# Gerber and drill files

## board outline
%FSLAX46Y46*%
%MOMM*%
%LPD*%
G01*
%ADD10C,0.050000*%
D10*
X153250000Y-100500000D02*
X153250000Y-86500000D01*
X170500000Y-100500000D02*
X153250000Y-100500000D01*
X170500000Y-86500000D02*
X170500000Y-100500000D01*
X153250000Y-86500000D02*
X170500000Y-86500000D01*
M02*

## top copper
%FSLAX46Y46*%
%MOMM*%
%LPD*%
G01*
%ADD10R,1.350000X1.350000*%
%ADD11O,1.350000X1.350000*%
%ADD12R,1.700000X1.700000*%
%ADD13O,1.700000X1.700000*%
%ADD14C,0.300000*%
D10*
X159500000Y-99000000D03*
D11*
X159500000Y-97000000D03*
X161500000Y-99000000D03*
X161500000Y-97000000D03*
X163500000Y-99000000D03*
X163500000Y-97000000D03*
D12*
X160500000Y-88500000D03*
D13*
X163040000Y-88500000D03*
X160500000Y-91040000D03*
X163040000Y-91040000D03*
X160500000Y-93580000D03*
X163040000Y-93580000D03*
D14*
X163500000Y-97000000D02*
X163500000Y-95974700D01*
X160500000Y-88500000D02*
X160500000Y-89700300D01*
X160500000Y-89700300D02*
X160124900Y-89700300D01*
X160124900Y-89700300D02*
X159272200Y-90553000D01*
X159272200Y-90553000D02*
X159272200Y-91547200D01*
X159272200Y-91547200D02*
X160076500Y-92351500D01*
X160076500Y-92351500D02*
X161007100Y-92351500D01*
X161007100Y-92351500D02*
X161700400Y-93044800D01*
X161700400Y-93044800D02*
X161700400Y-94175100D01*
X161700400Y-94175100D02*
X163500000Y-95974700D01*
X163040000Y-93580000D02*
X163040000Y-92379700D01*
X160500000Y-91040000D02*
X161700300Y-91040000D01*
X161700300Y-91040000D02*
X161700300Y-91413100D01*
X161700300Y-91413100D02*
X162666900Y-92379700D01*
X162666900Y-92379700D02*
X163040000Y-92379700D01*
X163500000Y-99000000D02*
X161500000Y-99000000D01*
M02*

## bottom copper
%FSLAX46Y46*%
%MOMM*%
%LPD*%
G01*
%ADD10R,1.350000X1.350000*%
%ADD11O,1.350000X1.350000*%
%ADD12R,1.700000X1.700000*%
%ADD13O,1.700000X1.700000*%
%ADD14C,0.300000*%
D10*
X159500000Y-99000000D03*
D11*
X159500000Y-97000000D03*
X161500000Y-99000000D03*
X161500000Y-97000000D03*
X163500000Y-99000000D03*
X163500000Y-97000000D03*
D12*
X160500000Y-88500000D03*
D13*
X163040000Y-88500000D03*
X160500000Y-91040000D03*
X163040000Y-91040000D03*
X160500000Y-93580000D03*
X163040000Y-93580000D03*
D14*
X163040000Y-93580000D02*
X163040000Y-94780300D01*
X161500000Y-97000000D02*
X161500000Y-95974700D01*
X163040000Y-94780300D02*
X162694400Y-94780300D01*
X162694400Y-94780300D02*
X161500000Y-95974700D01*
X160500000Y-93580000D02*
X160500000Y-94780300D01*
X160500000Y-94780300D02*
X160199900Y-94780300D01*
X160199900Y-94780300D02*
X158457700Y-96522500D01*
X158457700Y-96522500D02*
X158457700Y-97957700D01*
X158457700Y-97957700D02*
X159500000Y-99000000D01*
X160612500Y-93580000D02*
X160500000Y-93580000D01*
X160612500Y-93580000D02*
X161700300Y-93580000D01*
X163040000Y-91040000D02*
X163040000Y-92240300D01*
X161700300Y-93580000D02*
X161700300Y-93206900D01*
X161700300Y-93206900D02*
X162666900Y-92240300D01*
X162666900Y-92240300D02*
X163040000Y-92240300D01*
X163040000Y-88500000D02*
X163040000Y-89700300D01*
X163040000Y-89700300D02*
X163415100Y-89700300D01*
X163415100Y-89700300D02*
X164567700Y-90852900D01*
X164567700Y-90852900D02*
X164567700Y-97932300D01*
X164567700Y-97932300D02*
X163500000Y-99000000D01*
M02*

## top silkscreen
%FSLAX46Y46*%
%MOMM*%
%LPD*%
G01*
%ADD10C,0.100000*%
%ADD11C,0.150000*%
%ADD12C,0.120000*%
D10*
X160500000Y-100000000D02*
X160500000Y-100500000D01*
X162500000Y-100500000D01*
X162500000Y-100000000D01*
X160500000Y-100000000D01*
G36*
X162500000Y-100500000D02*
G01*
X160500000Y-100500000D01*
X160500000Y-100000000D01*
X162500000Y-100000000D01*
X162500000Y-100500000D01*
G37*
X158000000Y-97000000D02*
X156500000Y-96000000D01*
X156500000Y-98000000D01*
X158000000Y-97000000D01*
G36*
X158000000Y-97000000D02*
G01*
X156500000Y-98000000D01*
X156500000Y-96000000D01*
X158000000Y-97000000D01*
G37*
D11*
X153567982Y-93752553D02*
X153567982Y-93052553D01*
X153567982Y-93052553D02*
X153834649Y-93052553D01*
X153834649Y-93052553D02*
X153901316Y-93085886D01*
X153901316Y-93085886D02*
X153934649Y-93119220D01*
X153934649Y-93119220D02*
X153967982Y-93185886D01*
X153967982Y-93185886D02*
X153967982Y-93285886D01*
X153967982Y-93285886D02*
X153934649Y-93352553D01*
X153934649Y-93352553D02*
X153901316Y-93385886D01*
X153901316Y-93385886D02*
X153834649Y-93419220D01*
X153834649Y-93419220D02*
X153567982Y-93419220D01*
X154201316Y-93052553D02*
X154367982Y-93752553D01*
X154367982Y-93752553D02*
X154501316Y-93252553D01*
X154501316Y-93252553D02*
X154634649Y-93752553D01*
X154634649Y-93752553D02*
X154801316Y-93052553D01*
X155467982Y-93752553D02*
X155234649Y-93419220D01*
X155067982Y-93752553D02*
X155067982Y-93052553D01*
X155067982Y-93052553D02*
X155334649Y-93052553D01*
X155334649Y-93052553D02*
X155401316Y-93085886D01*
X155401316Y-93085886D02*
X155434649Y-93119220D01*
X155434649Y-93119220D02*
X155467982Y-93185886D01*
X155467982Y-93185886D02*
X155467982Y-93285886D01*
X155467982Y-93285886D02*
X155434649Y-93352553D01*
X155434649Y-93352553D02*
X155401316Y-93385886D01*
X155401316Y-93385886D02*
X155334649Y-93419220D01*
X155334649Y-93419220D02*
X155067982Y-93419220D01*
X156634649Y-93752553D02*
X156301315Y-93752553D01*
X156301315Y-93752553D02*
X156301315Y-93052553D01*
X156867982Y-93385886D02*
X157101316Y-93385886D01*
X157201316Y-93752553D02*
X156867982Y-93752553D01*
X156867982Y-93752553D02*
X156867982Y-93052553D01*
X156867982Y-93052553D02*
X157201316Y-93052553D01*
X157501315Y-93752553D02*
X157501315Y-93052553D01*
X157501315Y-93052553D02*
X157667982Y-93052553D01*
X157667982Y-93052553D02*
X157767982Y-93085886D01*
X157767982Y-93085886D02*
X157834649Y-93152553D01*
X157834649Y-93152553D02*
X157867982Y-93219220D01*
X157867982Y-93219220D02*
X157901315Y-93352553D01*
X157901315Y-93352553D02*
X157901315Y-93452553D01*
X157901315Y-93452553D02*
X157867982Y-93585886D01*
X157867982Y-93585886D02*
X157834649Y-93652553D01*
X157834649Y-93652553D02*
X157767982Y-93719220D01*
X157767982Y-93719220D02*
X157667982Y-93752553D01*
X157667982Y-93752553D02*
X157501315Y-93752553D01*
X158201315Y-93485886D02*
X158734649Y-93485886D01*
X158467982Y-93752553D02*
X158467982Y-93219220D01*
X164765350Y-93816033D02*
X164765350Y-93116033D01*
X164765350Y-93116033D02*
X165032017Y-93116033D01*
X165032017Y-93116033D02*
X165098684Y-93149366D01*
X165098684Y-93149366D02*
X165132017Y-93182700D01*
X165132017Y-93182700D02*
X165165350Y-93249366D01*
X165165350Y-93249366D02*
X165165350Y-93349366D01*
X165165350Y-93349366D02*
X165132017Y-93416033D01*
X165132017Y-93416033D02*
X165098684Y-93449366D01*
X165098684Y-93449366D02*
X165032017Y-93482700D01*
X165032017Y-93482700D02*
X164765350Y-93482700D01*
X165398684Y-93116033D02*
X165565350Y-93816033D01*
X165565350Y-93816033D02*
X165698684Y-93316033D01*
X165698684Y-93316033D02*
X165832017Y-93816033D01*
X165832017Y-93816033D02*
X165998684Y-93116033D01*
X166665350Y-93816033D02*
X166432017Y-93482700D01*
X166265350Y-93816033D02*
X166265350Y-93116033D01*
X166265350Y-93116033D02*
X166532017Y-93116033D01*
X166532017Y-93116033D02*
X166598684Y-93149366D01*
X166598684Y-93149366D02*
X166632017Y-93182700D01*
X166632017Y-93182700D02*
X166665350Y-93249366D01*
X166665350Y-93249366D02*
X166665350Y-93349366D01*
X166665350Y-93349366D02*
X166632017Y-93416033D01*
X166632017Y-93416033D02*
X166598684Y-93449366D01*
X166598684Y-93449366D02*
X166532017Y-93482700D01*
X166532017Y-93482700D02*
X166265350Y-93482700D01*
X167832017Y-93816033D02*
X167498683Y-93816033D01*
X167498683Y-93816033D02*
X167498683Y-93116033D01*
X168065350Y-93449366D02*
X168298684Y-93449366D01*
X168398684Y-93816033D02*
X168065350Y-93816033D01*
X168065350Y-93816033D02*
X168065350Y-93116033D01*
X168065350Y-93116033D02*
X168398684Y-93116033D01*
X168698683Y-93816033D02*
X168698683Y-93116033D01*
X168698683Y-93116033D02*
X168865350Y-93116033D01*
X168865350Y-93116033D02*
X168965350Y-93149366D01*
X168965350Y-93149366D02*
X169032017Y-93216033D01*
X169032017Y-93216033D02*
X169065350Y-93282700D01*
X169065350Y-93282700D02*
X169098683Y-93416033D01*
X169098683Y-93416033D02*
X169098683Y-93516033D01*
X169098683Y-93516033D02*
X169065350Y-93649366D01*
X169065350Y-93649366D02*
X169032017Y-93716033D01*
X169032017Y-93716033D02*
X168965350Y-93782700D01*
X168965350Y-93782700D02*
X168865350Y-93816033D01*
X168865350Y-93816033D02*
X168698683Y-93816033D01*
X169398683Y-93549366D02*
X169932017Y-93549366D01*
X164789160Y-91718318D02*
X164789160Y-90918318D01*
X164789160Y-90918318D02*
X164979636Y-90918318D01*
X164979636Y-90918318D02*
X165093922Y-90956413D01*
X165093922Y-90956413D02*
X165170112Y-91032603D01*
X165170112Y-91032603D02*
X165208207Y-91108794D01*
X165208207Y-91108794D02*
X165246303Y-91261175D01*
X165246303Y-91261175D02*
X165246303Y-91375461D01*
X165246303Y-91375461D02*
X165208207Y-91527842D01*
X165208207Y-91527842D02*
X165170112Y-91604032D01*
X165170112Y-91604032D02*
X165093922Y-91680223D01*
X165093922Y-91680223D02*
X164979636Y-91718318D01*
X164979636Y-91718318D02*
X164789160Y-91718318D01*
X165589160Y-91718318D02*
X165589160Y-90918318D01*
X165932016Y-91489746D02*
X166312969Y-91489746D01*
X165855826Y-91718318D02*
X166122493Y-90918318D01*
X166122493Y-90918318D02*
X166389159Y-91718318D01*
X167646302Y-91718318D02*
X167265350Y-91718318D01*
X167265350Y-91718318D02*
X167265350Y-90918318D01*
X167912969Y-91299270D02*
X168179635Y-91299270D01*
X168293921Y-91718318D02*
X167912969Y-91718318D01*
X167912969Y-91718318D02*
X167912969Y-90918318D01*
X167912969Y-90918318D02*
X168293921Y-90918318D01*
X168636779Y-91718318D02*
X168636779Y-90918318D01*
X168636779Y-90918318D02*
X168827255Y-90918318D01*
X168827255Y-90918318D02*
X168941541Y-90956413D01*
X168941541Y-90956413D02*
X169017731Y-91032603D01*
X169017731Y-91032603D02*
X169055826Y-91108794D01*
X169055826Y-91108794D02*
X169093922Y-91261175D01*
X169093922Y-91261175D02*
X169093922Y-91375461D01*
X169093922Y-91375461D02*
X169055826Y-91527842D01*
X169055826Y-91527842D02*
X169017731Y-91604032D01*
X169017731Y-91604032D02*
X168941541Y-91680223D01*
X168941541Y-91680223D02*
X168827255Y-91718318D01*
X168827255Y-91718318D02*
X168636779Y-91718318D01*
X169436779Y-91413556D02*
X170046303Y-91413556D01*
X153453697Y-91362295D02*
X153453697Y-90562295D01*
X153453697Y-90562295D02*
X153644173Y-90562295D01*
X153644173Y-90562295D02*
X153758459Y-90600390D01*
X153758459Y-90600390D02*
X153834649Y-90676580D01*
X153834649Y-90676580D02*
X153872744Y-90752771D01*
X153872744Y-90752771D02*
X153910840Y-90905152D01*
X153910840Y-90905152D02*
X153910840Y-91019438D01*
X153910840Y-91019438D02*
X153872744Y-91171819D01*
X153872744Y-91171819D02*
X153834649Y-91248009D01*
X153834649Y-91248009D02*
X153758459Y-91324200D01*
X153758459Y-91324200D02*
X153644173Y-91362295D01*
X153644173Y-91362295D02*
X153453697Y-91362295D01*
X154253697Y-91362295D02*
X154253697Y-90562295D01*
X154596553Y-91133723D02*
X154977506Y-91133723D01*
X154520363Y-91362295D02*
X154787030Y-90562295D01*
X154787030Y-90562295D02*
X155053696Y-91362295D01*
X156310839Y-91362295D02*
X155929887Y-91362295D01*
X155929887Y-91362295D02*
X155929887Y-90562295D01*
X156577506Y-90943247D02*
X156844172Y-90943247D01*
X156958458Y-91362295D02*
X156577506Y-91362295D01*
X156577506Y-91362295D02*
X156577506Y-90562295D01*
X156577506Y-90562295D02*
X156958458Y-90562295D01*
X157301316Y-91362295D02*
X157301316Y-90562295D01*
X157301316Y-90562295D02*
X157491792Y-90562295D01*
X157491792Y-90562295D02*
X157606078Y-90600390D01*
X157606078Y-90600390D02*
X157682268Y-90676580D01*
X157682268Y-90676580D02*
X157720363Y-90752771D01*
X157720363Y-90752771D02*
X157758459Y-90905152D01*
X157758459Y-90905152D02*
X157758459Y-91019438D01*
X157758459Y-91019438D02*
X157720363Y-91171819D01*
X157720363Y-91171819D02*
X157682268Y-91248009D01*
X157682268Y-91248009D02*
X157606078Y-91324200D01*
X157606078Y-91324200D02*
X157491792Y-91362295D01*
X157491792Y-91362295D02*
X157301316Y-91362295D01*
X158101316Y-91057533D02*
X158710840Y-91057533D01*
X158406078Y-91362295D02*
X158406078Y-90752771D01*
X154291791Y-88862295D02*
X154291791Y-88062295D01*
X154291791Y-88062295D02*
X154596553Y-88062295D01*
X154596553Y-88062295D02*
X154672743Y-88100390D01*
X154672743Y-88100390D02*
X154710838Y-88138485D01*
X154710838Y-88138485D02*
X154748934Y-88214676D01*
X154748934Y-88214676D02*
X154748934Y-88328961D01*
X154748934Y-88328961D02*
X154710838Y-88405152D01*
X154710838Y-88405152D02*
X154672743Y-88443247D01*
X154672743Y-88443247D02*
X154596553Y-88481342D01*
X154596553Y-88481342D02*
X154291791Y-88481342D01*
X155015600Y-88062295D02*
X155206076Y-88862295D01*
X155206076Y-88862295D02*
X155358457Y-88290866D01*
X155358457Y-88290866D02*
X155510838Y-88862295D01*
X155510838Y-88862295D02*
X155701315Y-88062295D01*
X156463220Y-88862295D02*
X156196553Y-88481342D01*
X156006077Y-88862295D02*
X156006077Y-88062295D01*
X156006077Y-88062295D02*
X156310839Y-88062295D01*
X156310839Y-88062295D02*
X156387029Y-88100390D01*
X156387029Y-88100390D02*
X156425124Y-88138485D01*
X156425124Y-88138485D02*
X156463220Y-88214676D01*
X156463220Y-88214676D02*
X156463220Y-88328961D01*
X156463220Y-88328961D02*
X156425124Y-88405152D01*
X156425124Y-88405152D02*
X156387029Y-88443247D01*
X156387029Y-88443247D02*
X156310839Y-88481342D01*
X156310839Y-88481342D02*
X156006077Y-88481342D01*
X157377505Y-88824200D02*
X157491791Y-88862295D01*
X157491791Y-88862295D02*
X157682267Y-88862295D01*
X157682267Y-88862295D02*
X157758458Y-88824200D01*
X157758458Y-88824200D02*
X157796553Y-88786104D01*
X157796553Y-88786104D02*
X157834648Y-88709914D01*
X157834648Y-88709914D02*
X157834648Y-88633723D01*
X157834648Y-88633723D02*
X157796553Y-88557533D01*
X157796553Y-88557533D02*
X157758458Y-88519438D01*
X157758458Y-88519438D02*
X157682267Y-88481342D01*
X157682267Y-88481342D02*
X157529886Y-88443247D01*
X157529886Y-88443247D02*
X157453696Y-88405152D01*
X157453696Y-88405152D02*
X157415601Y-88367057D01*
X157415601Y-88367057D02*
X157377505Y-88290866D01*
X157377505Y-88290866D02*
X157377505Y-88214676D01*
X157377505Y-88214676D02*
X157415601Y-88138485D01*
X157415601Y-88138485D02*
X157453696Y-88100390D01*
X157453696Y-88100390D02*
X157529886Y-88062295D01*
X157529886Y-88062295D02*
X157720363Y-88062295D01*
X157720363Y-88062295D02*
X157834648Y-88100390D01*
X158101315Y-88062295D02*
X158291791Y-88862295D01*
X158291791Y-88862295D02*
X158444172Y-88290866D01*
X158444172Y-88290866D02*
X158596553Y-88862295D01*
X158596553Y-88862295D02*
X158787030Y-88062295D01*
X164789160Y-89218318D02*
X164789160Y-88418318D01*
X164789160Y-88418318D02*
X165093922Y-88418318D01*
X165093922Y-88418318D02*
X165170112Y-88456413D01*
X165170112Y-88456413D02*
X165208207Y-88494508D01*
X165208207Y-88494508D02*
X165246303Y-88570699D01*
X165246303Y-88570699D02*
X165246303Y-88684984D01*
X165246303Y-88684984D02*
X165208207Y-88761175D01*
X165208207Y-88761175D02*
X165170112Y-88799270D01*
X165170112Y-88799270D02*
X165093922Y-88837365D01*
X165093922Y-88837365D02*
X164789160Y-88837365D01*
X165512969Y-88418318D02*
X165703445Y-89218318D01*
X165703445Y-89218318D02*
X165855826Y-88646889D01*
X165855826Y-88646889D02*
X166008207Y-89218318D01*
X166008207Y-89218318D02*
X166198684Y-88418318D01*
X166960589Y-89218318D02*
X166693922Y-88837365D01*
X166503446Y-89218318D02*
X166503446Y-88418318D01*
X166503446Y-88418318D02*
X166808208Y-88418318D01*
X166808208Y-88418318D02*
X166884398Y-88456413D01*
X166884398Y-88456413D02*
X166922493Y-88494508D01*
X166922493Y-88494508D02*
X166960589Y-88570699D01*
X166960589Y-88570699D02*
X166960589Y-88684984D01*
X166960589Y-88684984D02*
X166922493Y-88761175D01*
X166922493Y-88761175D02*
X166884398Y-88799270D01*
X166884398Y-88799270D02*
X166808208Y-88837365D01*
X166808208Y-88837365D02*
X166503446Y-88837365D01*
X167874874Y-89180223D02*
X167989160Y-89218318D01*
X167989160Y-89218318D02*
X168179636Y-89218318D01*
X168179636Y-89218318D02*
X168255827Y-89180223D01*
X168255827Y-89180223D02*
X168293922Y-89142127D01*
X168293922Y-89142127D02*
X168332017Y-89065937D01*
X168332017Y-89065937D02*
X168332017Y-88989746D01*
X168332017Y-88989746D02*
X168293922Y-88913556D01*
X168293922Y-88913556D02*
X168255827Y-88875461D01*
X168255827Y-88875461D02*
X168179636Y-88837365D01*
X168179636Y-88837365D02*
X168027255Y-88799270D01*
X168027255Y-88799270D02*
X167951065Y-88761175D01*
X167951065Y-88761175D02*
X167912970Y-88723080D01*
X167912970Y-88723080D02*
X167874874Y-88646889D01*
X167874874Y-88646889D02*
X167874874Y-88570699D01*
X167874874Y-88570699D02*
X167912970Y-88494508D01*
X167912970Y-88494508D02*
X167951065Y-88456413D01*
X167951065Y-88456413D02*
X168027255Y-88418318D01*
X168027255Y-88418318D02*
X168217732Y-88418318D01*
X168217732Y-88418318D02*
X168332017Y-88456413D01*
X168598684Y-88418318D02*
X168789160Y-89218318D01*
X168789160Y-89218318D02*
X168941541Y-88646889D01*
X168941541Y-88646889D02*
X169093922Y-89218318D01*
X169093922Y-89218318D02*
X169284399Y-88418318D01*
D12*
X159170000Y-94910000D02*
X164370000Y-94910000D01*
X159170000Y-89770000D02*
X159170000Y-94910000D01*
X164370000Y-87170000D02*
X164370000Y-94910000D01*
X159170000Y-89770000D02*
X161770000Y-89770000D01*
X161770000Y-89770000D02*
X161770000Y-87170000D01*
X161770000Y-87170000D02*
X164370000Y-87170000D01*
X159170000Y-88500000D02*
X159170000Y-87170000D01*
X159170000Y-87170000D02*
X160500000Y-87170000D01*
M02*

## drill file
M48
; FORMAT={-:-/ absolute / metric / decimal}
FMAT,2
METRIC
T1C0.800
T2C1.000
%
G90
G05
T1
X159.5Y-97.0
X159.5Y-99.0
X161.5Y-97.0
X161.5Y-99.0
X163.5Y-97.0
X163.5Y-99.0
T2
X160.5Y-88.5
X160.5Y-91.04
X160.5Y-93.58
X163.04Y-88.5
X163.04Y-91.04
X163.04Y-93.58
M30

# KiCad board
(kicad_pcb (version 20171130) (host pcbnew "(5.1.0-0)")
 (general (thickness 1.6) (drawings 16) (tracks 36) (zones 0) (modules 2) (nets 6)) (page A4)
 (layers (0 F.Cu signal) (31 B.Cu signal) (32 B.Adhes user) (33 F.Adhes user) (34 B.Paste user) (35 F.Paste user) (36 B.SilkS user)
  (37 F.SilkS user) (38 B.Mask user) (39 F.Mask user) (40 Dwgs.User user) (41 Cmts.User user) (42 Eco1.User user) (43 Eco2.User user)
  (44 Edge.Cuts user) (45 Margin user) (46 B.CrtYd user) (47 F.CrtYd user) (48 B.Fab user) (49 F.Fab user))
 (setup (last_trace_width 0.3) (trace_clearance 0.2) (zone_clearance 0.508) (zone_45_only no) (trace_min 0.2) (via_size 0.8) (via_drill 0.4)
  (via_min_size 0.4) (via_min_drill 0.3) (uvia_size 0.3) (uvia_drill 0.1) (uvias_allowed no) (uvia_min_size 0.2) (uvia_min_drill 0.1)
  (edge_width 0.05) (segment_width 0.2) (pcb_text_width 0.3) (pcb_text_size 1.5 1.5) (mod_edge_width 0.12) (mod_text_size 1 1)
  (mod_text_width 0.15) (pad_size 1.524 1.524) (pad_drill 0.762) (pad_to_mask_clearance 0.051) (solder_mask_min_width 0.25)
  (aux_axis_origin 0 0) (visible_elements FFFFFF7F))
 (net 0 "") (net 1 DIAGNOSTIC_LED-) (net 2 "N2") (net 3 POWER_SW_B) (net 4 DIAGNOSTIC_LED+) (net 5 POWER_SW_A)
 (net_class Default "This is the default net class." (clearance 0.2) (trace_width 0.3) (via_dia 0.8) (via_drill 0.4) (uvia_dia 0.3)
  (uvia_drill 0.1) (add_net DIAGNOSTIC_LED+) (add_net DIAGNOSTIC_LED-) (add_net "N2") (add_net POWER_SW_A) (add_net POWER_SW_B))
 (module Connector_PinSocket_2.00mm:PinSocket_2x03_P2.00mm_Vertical (layer B.Cu) (at 159.5 99 270)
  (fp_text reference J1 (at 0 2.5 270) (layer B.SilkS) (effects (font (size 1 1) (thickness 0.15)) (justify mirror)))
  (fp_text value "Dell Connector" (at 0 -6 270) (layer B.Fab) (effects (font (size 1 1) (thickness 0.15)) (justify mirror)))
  (pad 1 thru_hole rect (at 0 0 270) (size 1.35 1.35) (drill 0.8) (layers *.Cu *.Mask) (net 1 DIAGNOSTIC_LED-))
  (pad 2 thru_hole oval (at -2 0 270) (size 1.35 1.35) (drill 0.8) (layers *.Cu *.Mask) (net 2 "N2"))
  (pad 3 thru_hole oval (at 0 -2 270) (size 1.35 1.35) (drill 0.8) (layers *.Cu *.Mask) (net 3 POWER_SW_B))
  (pad 4 thru_hole oval (at -2 -2 270) (size 1.35 1.35) (drill 0.8) (layers *.Cu *.Mask) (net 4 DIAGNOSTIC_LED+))
  (pad 5 thru_hole oval (at 0 -4 270) (size 1.35 1.35) (drill 0.8) (layers *.Cu *.Mask) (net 3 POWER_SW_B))
  (pad 6 thru_hole oval (at -2 -4 270) (size 1.35 1.35) (drill 0.8) (layers *.Cu *.Mask) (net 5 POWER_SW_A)))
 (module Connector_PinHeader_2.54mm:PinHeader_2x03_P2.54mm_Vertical (layer F.Cu) (at 160.5 88.5)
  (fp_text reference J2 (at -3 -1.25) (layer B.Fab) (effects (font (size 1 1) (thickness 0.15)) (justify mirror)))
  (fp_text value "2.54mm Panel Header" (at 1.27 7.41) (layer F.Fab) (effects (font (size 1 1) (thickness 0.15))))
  (fp_line (start -1.33 6.41) (end 3.87 6.41) (layer F.SilkS) (width 0.12))
  (fp_line (start -1.33 1.27) (end -1.33 6.41) (layer F.SilkS) (width 0.12))
  (fp_line (start 3.87 -1.33) (end 3.87 6.41) (layer F.SilkS) (width 0.12))
  (fp_line (start -1.33 1.27) (end 1.27 1.27) (layer F.SilkS) (width 0.12))
  (fp_line (start 1.27 1.27) (end 1.27 -1.33) (layer F.SilkS) (width 0.12))
  (fp_line (start 1.27 -1.33) (end 3.87 -1.33) (layer F.SilkS) (width 0.12))
  (fp_line (start -1.33 0) (end -1.33 -1.33) (layer F.SilkS) (width 0.12))
  (fp_line (start -1.33 -1.33) (end 0 -1.33) (layer F.SilkS) (width 0.12))
  (pad 1 thru_hole rect (at 0 0) (size 1.7 1.7) (drill 1) (layers *.Cu *.Mask) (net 5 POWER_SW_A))
  (pad 2 thru_hole oval (at 2.54 0) (size 1.7 1.7) (drill 1) (layers *.Cu *.Mask) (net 3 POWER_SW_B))
  (pad 3 thru_hole oval (at 0 2.54) (size 1.7 1.7) (drill 1) (layers *.Cu *.Mask) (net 4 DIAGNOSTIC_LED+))
  (pad 4 thru_hole oval (at 2.54 2.54) (size 1.7 1.7) (drill 1) (layers *.Cu *.Mask) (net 1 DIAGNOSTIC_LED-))
  (pad 5 thru_hole oval (at 0 5.08) (size 1.7 1.7) (drill 1) (layers *.Cu *.Mask) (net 1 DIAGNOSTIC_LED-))
  (pad 6 thru_hole oval (at 2.54 5.08) (size 1.7 1.7) (drill 1) (layers *.Cu *.Mask) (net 4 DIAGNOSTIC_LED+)))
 (gr_poly (pts (xy 160.5 100) (xy 160.5 100.5) (xy 162.5 100.5) (xy 162.5 100)) (layer F.SilkS) (width 0.1))
 (gr_poly (pts (xy 158 97) (xy 156.5 96) (xy 156.5 98)) (layer F.SilkS) (width 0.1))
 (gr_line (start 153.25 100.5) (end 153.25 86.5) (layer Edge.Cuts) (width 0.05))
 (gr_line (start 170.5 100.5) (end 153.25 100.5) (layer Edge.Cuts) (width 0.05))
 (gr_line (start 170.5 86.5) (end 170.5 100.5) (layer Edge.Cuts) (width 0.05))
 (gr_line (start 153.25 86.5) (end 170.5 86.5) (layer Edge.Cuts) (width 0.05))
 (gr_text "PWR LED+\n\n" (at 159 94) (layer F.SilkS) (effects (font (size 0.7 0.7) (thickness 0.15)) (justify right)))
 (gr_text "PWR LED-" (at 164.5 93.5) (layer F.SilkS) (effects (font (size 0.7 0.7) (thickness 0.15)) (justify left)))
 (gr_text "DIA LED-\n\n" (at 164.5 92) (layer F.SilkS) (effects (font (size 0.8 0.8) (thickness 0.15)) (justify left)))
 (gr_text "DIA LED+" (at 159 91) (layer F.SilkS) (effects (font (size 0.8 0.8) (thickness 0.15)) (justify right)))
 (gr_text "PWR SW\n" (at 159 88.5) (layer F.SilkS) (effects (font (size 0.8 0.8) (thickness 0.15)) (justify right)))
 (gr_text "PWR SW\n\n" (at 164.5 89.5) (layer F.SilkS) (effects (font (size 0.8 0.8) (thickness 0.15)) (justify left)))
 (segment (start 163.5 97) (end 163.5 95.9747) (width 0.3) (layer F.Cu) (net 5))
 (segment (start 160.5 88.5) (end 160.5 89.7003) (width 0.3) (layer F.Cu) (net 5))
 (segment (start 160.5 89.7003) (end 160.1249 89.7003) (width 0.3) (layer F.Cu) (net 5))
 (segment (start 160.1249 89.7003) (end 159.2722 90.553) (width 0.3) (layer F.Cu) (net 5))
 (segment (start 159.2722 90.553) (end 159.2722 91.5472) (width 0.3) (layer F.Cu) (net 5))
 (segment (start 159.2722 91.5472) (end 160.0765 92.3515) (width 0.3) (layer F.Cu) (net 5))
 (segment (start 160.0765 92.3515) (end 161.0071 92.3515) (width 0.3) (layer F.Cu) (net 5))
 (segment (start 161.0071 92.3515) (end 161.7004 93.0448) (width 0.3) (layer F.Cu) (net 5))
 (segment (start 161.7004 93.0448) (end 161.7004 94.1751) (width 0.3) (layer F.Cu) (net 5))
 (segment (start 161.7004 94.1751) (end 163.5 95.9747) (width 0.3) (layer F.Cu) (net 5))
 (segment (start 163.04 93.58) (end 163.04 92.3797) (width 0.3) (layer F.Cu) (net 4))
 (segment (start 160.5 91.04) (end 161.7003 91.04) (width 0.3) (layer F.Cu) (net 4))
 (segment (start 161.7003 91.04) (end 161.7003 91.4131) (width 0.3) (layer F.Cu) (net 4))
 (segment (start 161.7003 91.4131) (end 162.6669 92.3797) (width 0.3) (layer F.Cu) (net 4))
 (segment (start 162.6669 92.3797) (end 163.04 92.3797) (width 0.3) (layer F.Cu) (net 4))
 (segment (start 163.04 93.58) (end 163.04 94.7803) (width 0.3) (layer B.Cu) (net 4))
 (segment (start 161.5 97) (end 161.5 95.9747) (width 0.3) (layer B.Cu) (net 4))
 (segment (start 163.04 94.7803) (end 162.6944 94.7803) (width 0.3) (layer B.Cu) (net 4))
 (segment (start 162.6944 94.7803) (end 161.5 95.9747) (width 0.3) (layer B.Cu) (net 4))
 (segment (start 160.5 93.58) (end 160.5 94.7803) (width 0.3) (layer B.Cu) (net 1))
 (segment (start 160.5 94.7803) (end 160.1999 94.7803) (width 0.3) (layer B.Cu) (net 1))
 (segment (start 160.1999 94.7803) (end 158.4577 96.5225) (width 0.3) (layer B.Cu) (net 1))
 (segment (start 158.4577 96.5225) (end 158.4577 97.9577) (width 0.3) (layer B.Cu) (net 1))
 (segment (start 158.4577 97.9577) (end 159.5 99) (width 0.3) (layer B.Cu) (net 1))
 (segment (start 160.6125 93.58) (end 160.5 93.58) (width 0.3) (layer B.Cu) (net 1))
 (segment (start 160.6125 93.58) (end 161.7003 93.58) (width 0.3) (layer B.Cu) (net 1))
 (segment (start 163.04 91.04) (end 163.04 92.2403) (width 0.3) (layer B.Cu) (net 1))
 (segment (start 161.7003 93.58) (end 161.7003 93.2069) (width 0.3) (layer B.Cu) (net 1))
 (segment (start 161.7003 93.2069) (end 162.6669 92.2403) (width 0.3) (layer B.Cu) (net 1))
 (segment (start 162.6669 92.2403) (end 163.04 92.2403) (width 0.3) (layer B.Cu) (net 1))
 (segment (start 163.5 99) (end 161.5 99) (width 0.3) (layer F.Cu) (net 3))
 (segment (start 163.04 88.5) (end 163.04 89.7003) (width 0.3) (layer B.Cu) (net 3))
 (segment (start 163.04 89.7003) (end 163.4151 89.7003) (width 0.3) (layer B.Cu) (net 3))
 (segment (start 163.4151 89.7003) (end 164.5677 90.8529) (width 0.3) (layer B.Cu) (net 3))
 (segment (start 164.5677 90.8529) (end 164.5677 97.9323) (width 0.3) (layer B.Cu) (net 3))
 (segment (start 164.5677 97.9323) (end 163.5 99) (width 0.3) (layer B.Cu) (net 3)))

